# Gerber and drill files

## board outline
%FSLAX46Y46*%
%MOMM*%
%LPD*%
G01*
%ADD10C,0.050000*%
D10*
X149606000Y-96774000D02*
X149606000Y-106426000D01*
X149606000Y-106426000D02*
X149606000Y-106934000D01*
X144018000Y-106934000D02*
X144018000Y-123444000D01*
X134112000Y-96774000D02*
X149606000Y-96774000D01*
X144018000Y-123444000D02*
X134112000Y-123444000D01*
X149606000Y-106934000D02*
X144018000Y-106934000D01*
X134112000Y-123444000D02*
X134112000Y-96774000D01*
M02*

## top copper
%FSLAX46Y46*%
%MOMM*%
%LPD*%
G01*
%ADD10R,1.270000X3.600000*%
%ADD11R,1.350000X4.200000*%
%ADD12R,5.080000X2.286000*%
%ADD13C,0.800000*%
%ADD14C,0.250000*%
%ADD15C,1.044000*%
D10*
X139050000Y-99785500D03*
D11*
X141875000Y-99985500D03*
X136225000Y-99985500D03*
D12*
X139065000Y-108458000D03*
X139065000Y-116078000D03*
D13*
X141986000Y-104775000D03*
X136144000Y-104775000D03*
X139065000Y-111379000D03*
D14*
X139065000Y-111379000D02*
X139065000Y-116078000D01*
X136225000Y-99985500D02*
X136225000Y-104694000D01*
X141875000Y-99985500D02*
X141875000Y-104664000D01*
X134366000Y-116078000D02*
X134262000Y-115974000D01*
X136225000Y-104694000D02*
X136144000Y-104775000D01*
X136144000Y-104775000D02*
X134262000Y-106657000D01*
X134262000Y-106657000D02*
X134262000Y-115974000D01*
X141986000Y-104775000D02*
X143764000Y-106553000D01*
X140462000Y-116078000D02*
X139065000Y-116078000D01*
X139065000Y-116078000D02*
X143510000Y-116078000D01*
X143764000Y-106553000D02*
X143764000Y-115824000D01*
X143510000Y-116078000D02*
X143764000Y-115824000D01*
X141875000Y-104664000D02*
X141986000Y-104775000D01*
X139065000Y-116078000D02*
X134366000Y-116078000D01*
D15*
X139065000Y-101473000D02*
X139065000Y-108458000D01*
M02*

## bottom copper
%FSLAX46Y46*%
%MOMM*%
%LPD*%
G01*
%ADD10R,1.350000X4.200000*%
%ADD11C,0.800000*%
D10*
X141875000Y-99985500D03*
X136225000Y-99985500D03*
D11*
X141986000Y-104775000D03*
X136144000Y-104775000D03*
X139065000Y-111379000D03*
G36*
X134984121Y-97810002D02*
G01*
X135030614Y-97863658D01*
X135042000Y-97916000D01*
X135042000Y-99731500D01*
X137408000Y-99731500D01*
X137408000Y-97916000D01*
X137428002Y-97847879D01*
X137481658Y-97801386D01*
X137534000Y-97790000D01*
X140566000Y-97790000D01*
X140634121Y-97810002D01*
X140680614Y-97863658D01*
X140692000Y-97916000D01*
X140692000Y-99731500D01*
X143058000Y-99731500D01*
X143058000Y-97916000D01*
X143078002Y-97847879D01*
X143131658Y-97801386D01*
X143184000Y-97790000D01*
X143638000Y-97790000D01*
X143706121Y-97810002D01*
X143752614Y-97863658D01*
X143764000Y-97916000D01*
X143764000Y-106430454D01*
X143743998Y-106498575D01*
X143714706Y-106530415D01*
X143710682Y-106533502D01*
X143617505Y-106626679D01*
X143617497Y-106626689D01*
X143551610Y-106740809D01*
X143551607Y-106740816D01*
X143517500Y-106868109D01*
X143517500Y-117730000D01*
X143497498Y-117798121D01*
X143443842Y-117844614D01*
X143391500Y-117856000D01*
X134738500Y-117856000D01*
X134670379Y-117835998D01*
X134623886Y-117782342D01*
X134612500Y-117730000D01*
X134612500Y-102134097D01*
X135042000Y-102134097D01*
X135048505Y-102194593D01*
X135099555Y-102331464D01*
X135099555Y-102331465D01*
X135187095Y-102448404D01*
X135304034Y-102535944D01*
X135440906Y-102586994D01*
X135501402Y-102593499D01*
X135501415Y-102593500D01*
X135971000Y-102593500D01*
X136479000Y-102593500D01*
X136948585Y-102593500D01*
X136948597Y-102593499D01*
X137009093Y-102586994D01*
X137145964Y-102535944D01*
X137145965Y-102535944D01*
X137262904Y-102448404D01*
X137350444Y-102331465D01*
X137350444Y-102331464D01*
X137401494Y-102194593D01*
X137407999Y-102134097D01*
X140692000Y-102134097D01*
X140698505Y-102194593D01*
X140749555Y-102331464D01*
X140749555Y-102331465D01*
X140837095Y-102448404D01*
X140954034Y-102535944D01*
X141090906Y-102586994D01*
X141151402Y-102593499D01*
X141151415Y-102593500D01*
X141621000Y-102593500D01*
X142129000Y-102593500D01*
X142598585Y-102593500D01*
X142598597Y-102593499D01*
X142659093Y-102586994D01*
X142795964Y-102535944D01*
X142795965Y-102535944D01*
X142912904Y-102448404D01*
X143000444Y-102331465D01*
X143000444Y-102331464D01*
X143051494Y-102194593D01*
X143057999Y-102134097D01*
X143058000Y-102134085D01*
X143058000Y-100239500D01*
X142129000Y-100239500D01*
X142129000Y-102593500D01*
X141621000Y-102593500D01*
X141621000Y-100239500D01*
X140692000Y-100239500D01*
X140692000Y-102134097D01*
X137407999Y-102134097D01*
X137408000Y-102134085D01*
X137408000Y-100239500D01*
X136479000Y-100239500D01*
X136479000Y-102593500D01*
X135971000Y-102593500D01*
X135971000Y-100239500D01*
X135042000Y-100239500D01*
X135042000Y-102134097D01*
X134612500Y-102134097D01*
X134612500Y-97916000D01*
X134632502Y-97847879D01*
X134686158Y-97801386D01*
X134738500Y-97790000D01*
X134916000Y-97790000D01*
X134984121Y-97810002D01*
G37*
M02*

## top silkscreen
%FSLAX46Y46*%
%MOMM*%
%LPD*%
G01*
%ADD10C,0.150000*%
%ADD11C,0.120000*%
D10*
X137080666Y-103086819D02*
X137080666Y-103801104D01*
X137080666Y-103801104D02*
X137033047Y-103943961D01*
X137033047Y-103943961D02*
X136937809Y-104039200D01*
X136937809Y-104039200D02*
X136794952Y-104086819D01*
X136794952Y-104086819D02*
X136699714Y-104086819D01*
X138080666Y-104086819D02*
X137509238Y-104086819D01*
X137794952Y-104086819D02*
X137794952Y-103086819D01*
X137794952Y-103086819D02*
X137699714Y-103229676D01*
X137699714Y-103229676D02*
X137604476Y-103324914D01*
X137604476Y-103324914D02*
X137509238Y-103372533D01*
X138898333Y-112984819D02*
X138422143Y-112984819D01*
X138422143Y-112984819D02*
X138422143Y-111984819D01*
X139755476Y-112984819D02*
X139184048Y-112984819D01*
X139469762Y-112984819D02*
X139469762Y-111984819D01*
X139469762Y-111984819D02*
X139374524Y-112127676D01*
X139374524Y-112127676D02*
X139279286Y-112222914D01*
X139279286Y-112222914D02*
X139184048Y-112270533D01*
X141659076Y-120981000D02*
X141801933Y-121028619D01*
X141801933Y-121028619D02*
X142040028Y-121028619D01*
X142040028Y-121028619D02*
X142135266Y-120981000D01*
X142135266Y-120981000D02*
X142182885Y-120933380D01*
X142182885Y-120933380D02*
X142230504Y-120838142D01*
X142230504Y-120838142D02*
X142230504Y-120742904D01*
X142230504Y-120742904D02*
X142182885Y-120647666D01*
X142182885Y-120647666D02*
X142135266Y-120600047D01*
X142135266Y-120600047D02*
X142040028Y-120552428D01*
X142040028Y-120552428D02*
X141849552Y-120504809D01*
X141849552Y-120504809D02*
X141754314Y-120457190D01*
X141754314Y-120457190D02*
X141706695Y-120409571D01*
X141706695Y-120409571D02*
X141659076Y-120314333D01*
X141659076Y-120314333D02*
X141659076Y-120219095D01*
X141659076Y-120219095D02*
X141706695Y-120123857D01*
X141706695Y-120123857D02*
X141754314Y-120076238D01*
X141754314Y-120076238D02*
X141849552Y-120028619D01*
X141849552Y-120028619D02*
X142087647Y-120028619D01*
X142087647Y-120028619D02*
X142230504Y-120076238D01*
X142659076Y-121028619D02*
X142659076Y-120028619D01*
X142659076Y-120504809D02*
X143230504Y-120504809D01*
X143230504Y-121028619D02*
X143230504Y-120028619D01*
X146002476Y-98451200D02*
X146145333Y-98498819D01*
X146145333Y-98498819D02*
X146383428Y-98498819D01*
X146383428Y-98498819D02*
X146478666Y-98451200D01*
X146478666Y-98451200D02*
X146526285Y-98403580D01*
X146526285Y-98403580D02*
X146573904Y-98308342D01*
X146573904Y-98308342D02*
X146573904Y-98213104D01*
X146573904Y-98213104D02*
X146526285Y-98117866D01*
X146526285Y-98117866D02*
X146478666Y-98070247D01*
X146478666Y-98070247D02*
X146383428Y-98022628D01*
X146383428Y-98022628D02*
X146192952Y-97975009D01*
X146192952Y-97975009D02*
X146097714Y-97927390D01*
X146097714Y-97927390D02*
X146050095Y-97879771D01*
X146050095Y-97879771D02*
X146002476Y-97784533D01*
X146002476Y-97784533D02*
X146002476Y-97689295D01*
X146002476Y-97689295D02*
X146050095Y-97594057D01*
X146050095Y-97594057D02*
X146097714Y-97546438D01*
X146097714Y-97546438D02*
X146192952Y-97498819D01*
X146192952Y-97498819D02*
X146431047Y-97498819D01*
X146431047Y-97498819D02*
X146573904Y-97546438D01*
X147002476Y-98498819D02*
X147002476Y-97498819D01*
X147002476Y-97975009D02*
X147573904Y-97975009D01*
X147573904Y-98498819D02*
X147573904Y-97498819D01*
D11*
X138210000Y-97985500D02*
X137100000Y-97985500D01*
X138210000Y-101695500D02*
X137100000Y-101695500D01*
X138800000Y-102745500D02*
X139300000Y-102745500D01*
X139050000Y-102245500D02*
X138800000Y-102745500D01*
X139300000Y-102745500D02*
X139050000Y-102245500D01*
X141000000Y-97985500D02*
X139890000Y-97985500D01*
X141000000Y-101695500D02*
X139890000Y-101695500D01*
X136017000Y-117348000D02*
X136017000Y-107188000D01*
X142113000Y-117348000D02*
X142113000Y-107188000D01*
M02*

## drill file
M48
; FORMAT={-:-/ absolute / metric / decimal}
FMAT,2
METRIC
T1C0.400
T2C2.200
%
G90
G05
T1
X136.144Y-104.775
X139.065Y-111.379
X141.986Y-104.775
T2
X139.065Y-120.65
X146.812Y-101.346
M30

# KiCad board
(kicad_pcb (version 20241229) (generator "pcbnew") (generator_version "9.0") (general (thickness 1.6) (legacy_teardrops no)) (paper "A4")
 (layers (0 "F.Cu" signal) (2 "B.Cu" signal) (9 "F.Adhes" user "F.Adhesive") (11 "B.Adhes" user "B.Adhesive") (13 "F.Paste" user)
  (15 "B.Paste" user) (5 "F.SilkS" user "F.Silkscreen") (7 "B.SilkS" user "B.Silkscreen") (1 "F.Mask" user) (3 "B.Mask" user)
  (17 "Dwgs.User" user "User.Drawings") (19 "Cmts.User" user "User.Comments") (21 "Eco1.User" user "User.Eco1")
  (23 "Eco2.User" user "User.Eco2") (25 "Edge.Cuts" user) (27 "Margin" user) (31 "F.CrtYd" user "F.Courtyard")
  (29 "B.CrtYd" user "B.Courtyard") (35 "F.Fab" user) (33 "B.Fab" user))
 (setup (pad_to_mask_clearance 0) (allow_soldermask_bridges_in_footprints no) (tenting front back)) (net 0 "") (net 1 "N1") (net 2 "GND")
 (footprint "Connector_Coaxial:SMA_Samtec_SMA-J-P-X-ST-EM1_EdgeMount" (layer "F.Cu") (at 139.05 99.9855 180)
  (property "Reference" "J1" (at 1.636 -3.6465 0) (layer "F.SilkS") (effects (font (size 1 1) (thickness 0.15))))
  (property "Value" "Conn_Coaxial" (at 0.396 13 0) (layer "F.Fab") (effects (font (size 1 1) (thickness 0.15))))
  (fp_line (start 0.84 2) (end 1.95 2) (stroke (width 0.12) (type solid)) (layer "F.SilkS"))
  (fp_line (start 0.84 -1.71) (end 1.95 -1.71) (stroke (width 0.12) (type solid)) (layer "F.SilkS"))
  (fp_line (start 0.25 -2.76) (end -0.25 -2.76) (stroke (width 0.12) (type solid)) (layer "F.SilkS"))
  (fp_line (start 0 -2.26) (end 0.25 -2.76) (stroke (width 0.12) (type solid)) (layer "F.SilkS"))
  (fp_line (start -0.25 -2.76) (end 0 -2.26) (stroke (width 0.12) (type solid)) (layer "F.SilkS"))
  (fp_line (start -1.95 2) (end -0.84 2) (stroke (width 0.12) (type solid)) (layer "F.SilkS"))
  (fp_line (start -1.95 -1.71) (end -0.84 -1.71) (stroke (width 0.12) (type solid)) (layer "F.SilkS"))
  (pad "1" smd rect (at 0 0.2 180) (size 1.27 3.6) (layers "F.Cu" "F.Mask" "F.Paste") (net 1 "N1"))
  (pad "2" smd rect (at -2.825 0 180) (size 1.35 4.2) (layers "F.Cu" "F.Mask" "F.Paste") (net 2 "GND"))
  (pad "2" smd rect (at -2.825 0 180) (size 1.35 4.2) (layers "B.Cu" "B.Mask" "B.Paste") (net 2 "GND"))
  (pad "2" smd rect (at 2.825 0 180) (size 1.35 4.2) (layers "F.Cu" "F.Mask" "F.Paste") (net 2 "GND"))
  (pad "2" smd rect (at 2.825 0 180) (size 1.35 4.2) (layers "B.Cu" "B.Mask" "B.Paste") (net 2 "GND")))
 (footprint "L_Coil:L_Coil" (layer "F.Cu") (at 139.065 109.474 180)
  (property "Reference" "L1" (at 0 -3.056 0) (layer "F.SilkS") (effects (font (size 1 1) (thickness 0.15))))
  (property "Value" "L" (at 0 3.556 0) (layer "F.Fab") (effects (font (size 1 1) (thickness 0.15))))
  (fp_line (start 3.048 -7.874) (end 3.048 2.286) (stroke (width 0.12) (type solid)) (layer "F.SilkS"))
  (fp_line (start -3.048 -7.874) (end -3.048 2.286) (stroke (width 0.12) (type solid)) (layer "F.SilkS"))
  (pad "1" smd rect (at 0 1.016 180) (size 5.08 2.286) (layers "F.Cu" "F.Mask" "F.Paste") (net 1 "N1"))
  (pad "2" smd rect (at 0 -6.604 180) (size 5.08 2.286) (layers "F.Cu" "F.Mask" "F.Paste") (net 2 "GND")))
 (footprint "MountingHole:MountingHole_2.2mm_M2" (layer "F.Cu") (at 139.065 120.65)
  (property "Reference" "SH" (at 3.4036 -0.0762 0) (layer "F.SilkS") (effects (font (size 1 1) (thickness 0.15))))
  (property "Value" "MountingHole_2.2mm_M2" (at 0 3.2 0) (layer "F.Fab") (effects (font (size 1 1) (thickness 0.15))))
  (pad "" np_thru_hole circle (at 0 0) (size 2.2 2.2) (drill 2.2) (layers "*.Cu" "*.Mask")))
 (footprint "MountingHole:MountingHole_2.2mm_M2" (layer "F.Cu") (at 146.812 101.346)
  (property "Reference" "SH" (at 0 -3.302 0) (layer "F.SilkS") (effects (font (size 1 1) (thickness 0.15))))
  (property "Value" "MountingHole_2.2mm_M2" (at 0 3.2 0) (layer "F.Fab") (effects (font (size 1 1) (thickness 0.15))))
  (pad "" np_thru_hole circle (at 0 0) (size 2.2 2.2) (drill 2.2) (layers "*.Cu" "*.Mask")))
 (gr_line (start 149.606 96.774) (end 149.606 106.426) (stroke (width 0.05) (type solid)) (layer "Edge.Cuts"))
 (gr_line (start 149.606 106.426) (end 149.606 106.934) (stroke (width 0.05) (type solid)) (layer "Edge.Cuts"))
 (gr_line (start 144.018 106.934) (end 144.018 123.444) (stroke (width 0.05) (type solid)) (layer "Edge.Cuts"))
 (gr_line (start 134.112 96.774) (end 149.606 96.774) (stroke (width 0.05) (type solid)) (layer "Edge.Cuts"))
 (gr_line (start 144.018 123.444) (end 134.112 123.444) (stroke (width 0.05) (type solid)) (layer "Edge.Cuts"))
 (gr_line (start 149.606 106.934) (end 144.018 106.934) (stroke (width 0.05) (type solid)) (layer "Edge.Cuts"))
 (gr_line (start 134.112 123.444) (end 134.112 96.774) (stroke (width 0.05) (type solid)) (layer "Edge.Cuts"))
 (segment (start 139.065 111.379) (end 139.065 116.078) (width 0.25) (layer "F.Cu") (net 2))
 (segment (start 136.225 99.9855) (end 136.225 104.694) (width 0.25) (layer "F.Cu") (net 2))
 (segment (start 141.875 99.9855) (end 141.875 104.664) (width 0.25) (layer "F.Cu") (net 2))
 (segment (start 134.366 116.078) (end 134.262 115.974) (width 0.25) (layer "F.Cu") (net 2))
 (segment (start 136.225 104.694) (end 136.144 104.775) (width 0.25) (layer "F.Cu") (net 2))
 (segment (start 136.144 104.775) (end 134.262 106.657) (width 0.25) (layer "F.Cu") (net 2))
 (segment (start 134.262 106.657) (end 134.262 115.974) (width 0.25) (layer "F.Cu") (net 2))
 (segment (start 141.986 104.775) (end 143.764 106.553) (width 0.25) (layer "F.Cu") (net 2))
 (segment (start 140.462 116.078) (end 139.065 116.078) (width 0.25) (layer "F.Cu") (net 2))
 (segment (start 139.065 116.078) (end 143.51 116.078) (width 0.25) (layer "F.Cu") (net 2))
 (segment (start 143.764 106.553) (end 143.764 115.824) (width 0.25) (layer "F.Cu") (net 2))
 (segment (start 143.51 116.078) (end 143.764 115.824) (width 0.25) (layer "F.Cu") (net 2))
 (segment (start 141.875 104.664) (end 141.986 104.775) (width 0.25) (layer "F.Cu") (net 2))
 (segment (start 139.065 116.078) (end 134.366 116.078) (width 0.25) (layer "F.Cu") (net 2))
 (via (at 141.986 104.775) (size 0.8) (drill 0.4) (layers "F.Cu" "B.Cu") (free yes) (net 2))
 (via (at 136.144 104.775) (size 0.8) (drill 0.4) (layers "F.Cu" "B.Cu") (free yes) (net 2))
 (via (at 139.065 111.379) (size 0.8) (drill 0.4) (layers "F.Cu" "B.Cu") (free yes) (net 2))
 (segment (start 139.065 101.473) (end 139.065 108.458) (width 1.044) (layer "F.Cu") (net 1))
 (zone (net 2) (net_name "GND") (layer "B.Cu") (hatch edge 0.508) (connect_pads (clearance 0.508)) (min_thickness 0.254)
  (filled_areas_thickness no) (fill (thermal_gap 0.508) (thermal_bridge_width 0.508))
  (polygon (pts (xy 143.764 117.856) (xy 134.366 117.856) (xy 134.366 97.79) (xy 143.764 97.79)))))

